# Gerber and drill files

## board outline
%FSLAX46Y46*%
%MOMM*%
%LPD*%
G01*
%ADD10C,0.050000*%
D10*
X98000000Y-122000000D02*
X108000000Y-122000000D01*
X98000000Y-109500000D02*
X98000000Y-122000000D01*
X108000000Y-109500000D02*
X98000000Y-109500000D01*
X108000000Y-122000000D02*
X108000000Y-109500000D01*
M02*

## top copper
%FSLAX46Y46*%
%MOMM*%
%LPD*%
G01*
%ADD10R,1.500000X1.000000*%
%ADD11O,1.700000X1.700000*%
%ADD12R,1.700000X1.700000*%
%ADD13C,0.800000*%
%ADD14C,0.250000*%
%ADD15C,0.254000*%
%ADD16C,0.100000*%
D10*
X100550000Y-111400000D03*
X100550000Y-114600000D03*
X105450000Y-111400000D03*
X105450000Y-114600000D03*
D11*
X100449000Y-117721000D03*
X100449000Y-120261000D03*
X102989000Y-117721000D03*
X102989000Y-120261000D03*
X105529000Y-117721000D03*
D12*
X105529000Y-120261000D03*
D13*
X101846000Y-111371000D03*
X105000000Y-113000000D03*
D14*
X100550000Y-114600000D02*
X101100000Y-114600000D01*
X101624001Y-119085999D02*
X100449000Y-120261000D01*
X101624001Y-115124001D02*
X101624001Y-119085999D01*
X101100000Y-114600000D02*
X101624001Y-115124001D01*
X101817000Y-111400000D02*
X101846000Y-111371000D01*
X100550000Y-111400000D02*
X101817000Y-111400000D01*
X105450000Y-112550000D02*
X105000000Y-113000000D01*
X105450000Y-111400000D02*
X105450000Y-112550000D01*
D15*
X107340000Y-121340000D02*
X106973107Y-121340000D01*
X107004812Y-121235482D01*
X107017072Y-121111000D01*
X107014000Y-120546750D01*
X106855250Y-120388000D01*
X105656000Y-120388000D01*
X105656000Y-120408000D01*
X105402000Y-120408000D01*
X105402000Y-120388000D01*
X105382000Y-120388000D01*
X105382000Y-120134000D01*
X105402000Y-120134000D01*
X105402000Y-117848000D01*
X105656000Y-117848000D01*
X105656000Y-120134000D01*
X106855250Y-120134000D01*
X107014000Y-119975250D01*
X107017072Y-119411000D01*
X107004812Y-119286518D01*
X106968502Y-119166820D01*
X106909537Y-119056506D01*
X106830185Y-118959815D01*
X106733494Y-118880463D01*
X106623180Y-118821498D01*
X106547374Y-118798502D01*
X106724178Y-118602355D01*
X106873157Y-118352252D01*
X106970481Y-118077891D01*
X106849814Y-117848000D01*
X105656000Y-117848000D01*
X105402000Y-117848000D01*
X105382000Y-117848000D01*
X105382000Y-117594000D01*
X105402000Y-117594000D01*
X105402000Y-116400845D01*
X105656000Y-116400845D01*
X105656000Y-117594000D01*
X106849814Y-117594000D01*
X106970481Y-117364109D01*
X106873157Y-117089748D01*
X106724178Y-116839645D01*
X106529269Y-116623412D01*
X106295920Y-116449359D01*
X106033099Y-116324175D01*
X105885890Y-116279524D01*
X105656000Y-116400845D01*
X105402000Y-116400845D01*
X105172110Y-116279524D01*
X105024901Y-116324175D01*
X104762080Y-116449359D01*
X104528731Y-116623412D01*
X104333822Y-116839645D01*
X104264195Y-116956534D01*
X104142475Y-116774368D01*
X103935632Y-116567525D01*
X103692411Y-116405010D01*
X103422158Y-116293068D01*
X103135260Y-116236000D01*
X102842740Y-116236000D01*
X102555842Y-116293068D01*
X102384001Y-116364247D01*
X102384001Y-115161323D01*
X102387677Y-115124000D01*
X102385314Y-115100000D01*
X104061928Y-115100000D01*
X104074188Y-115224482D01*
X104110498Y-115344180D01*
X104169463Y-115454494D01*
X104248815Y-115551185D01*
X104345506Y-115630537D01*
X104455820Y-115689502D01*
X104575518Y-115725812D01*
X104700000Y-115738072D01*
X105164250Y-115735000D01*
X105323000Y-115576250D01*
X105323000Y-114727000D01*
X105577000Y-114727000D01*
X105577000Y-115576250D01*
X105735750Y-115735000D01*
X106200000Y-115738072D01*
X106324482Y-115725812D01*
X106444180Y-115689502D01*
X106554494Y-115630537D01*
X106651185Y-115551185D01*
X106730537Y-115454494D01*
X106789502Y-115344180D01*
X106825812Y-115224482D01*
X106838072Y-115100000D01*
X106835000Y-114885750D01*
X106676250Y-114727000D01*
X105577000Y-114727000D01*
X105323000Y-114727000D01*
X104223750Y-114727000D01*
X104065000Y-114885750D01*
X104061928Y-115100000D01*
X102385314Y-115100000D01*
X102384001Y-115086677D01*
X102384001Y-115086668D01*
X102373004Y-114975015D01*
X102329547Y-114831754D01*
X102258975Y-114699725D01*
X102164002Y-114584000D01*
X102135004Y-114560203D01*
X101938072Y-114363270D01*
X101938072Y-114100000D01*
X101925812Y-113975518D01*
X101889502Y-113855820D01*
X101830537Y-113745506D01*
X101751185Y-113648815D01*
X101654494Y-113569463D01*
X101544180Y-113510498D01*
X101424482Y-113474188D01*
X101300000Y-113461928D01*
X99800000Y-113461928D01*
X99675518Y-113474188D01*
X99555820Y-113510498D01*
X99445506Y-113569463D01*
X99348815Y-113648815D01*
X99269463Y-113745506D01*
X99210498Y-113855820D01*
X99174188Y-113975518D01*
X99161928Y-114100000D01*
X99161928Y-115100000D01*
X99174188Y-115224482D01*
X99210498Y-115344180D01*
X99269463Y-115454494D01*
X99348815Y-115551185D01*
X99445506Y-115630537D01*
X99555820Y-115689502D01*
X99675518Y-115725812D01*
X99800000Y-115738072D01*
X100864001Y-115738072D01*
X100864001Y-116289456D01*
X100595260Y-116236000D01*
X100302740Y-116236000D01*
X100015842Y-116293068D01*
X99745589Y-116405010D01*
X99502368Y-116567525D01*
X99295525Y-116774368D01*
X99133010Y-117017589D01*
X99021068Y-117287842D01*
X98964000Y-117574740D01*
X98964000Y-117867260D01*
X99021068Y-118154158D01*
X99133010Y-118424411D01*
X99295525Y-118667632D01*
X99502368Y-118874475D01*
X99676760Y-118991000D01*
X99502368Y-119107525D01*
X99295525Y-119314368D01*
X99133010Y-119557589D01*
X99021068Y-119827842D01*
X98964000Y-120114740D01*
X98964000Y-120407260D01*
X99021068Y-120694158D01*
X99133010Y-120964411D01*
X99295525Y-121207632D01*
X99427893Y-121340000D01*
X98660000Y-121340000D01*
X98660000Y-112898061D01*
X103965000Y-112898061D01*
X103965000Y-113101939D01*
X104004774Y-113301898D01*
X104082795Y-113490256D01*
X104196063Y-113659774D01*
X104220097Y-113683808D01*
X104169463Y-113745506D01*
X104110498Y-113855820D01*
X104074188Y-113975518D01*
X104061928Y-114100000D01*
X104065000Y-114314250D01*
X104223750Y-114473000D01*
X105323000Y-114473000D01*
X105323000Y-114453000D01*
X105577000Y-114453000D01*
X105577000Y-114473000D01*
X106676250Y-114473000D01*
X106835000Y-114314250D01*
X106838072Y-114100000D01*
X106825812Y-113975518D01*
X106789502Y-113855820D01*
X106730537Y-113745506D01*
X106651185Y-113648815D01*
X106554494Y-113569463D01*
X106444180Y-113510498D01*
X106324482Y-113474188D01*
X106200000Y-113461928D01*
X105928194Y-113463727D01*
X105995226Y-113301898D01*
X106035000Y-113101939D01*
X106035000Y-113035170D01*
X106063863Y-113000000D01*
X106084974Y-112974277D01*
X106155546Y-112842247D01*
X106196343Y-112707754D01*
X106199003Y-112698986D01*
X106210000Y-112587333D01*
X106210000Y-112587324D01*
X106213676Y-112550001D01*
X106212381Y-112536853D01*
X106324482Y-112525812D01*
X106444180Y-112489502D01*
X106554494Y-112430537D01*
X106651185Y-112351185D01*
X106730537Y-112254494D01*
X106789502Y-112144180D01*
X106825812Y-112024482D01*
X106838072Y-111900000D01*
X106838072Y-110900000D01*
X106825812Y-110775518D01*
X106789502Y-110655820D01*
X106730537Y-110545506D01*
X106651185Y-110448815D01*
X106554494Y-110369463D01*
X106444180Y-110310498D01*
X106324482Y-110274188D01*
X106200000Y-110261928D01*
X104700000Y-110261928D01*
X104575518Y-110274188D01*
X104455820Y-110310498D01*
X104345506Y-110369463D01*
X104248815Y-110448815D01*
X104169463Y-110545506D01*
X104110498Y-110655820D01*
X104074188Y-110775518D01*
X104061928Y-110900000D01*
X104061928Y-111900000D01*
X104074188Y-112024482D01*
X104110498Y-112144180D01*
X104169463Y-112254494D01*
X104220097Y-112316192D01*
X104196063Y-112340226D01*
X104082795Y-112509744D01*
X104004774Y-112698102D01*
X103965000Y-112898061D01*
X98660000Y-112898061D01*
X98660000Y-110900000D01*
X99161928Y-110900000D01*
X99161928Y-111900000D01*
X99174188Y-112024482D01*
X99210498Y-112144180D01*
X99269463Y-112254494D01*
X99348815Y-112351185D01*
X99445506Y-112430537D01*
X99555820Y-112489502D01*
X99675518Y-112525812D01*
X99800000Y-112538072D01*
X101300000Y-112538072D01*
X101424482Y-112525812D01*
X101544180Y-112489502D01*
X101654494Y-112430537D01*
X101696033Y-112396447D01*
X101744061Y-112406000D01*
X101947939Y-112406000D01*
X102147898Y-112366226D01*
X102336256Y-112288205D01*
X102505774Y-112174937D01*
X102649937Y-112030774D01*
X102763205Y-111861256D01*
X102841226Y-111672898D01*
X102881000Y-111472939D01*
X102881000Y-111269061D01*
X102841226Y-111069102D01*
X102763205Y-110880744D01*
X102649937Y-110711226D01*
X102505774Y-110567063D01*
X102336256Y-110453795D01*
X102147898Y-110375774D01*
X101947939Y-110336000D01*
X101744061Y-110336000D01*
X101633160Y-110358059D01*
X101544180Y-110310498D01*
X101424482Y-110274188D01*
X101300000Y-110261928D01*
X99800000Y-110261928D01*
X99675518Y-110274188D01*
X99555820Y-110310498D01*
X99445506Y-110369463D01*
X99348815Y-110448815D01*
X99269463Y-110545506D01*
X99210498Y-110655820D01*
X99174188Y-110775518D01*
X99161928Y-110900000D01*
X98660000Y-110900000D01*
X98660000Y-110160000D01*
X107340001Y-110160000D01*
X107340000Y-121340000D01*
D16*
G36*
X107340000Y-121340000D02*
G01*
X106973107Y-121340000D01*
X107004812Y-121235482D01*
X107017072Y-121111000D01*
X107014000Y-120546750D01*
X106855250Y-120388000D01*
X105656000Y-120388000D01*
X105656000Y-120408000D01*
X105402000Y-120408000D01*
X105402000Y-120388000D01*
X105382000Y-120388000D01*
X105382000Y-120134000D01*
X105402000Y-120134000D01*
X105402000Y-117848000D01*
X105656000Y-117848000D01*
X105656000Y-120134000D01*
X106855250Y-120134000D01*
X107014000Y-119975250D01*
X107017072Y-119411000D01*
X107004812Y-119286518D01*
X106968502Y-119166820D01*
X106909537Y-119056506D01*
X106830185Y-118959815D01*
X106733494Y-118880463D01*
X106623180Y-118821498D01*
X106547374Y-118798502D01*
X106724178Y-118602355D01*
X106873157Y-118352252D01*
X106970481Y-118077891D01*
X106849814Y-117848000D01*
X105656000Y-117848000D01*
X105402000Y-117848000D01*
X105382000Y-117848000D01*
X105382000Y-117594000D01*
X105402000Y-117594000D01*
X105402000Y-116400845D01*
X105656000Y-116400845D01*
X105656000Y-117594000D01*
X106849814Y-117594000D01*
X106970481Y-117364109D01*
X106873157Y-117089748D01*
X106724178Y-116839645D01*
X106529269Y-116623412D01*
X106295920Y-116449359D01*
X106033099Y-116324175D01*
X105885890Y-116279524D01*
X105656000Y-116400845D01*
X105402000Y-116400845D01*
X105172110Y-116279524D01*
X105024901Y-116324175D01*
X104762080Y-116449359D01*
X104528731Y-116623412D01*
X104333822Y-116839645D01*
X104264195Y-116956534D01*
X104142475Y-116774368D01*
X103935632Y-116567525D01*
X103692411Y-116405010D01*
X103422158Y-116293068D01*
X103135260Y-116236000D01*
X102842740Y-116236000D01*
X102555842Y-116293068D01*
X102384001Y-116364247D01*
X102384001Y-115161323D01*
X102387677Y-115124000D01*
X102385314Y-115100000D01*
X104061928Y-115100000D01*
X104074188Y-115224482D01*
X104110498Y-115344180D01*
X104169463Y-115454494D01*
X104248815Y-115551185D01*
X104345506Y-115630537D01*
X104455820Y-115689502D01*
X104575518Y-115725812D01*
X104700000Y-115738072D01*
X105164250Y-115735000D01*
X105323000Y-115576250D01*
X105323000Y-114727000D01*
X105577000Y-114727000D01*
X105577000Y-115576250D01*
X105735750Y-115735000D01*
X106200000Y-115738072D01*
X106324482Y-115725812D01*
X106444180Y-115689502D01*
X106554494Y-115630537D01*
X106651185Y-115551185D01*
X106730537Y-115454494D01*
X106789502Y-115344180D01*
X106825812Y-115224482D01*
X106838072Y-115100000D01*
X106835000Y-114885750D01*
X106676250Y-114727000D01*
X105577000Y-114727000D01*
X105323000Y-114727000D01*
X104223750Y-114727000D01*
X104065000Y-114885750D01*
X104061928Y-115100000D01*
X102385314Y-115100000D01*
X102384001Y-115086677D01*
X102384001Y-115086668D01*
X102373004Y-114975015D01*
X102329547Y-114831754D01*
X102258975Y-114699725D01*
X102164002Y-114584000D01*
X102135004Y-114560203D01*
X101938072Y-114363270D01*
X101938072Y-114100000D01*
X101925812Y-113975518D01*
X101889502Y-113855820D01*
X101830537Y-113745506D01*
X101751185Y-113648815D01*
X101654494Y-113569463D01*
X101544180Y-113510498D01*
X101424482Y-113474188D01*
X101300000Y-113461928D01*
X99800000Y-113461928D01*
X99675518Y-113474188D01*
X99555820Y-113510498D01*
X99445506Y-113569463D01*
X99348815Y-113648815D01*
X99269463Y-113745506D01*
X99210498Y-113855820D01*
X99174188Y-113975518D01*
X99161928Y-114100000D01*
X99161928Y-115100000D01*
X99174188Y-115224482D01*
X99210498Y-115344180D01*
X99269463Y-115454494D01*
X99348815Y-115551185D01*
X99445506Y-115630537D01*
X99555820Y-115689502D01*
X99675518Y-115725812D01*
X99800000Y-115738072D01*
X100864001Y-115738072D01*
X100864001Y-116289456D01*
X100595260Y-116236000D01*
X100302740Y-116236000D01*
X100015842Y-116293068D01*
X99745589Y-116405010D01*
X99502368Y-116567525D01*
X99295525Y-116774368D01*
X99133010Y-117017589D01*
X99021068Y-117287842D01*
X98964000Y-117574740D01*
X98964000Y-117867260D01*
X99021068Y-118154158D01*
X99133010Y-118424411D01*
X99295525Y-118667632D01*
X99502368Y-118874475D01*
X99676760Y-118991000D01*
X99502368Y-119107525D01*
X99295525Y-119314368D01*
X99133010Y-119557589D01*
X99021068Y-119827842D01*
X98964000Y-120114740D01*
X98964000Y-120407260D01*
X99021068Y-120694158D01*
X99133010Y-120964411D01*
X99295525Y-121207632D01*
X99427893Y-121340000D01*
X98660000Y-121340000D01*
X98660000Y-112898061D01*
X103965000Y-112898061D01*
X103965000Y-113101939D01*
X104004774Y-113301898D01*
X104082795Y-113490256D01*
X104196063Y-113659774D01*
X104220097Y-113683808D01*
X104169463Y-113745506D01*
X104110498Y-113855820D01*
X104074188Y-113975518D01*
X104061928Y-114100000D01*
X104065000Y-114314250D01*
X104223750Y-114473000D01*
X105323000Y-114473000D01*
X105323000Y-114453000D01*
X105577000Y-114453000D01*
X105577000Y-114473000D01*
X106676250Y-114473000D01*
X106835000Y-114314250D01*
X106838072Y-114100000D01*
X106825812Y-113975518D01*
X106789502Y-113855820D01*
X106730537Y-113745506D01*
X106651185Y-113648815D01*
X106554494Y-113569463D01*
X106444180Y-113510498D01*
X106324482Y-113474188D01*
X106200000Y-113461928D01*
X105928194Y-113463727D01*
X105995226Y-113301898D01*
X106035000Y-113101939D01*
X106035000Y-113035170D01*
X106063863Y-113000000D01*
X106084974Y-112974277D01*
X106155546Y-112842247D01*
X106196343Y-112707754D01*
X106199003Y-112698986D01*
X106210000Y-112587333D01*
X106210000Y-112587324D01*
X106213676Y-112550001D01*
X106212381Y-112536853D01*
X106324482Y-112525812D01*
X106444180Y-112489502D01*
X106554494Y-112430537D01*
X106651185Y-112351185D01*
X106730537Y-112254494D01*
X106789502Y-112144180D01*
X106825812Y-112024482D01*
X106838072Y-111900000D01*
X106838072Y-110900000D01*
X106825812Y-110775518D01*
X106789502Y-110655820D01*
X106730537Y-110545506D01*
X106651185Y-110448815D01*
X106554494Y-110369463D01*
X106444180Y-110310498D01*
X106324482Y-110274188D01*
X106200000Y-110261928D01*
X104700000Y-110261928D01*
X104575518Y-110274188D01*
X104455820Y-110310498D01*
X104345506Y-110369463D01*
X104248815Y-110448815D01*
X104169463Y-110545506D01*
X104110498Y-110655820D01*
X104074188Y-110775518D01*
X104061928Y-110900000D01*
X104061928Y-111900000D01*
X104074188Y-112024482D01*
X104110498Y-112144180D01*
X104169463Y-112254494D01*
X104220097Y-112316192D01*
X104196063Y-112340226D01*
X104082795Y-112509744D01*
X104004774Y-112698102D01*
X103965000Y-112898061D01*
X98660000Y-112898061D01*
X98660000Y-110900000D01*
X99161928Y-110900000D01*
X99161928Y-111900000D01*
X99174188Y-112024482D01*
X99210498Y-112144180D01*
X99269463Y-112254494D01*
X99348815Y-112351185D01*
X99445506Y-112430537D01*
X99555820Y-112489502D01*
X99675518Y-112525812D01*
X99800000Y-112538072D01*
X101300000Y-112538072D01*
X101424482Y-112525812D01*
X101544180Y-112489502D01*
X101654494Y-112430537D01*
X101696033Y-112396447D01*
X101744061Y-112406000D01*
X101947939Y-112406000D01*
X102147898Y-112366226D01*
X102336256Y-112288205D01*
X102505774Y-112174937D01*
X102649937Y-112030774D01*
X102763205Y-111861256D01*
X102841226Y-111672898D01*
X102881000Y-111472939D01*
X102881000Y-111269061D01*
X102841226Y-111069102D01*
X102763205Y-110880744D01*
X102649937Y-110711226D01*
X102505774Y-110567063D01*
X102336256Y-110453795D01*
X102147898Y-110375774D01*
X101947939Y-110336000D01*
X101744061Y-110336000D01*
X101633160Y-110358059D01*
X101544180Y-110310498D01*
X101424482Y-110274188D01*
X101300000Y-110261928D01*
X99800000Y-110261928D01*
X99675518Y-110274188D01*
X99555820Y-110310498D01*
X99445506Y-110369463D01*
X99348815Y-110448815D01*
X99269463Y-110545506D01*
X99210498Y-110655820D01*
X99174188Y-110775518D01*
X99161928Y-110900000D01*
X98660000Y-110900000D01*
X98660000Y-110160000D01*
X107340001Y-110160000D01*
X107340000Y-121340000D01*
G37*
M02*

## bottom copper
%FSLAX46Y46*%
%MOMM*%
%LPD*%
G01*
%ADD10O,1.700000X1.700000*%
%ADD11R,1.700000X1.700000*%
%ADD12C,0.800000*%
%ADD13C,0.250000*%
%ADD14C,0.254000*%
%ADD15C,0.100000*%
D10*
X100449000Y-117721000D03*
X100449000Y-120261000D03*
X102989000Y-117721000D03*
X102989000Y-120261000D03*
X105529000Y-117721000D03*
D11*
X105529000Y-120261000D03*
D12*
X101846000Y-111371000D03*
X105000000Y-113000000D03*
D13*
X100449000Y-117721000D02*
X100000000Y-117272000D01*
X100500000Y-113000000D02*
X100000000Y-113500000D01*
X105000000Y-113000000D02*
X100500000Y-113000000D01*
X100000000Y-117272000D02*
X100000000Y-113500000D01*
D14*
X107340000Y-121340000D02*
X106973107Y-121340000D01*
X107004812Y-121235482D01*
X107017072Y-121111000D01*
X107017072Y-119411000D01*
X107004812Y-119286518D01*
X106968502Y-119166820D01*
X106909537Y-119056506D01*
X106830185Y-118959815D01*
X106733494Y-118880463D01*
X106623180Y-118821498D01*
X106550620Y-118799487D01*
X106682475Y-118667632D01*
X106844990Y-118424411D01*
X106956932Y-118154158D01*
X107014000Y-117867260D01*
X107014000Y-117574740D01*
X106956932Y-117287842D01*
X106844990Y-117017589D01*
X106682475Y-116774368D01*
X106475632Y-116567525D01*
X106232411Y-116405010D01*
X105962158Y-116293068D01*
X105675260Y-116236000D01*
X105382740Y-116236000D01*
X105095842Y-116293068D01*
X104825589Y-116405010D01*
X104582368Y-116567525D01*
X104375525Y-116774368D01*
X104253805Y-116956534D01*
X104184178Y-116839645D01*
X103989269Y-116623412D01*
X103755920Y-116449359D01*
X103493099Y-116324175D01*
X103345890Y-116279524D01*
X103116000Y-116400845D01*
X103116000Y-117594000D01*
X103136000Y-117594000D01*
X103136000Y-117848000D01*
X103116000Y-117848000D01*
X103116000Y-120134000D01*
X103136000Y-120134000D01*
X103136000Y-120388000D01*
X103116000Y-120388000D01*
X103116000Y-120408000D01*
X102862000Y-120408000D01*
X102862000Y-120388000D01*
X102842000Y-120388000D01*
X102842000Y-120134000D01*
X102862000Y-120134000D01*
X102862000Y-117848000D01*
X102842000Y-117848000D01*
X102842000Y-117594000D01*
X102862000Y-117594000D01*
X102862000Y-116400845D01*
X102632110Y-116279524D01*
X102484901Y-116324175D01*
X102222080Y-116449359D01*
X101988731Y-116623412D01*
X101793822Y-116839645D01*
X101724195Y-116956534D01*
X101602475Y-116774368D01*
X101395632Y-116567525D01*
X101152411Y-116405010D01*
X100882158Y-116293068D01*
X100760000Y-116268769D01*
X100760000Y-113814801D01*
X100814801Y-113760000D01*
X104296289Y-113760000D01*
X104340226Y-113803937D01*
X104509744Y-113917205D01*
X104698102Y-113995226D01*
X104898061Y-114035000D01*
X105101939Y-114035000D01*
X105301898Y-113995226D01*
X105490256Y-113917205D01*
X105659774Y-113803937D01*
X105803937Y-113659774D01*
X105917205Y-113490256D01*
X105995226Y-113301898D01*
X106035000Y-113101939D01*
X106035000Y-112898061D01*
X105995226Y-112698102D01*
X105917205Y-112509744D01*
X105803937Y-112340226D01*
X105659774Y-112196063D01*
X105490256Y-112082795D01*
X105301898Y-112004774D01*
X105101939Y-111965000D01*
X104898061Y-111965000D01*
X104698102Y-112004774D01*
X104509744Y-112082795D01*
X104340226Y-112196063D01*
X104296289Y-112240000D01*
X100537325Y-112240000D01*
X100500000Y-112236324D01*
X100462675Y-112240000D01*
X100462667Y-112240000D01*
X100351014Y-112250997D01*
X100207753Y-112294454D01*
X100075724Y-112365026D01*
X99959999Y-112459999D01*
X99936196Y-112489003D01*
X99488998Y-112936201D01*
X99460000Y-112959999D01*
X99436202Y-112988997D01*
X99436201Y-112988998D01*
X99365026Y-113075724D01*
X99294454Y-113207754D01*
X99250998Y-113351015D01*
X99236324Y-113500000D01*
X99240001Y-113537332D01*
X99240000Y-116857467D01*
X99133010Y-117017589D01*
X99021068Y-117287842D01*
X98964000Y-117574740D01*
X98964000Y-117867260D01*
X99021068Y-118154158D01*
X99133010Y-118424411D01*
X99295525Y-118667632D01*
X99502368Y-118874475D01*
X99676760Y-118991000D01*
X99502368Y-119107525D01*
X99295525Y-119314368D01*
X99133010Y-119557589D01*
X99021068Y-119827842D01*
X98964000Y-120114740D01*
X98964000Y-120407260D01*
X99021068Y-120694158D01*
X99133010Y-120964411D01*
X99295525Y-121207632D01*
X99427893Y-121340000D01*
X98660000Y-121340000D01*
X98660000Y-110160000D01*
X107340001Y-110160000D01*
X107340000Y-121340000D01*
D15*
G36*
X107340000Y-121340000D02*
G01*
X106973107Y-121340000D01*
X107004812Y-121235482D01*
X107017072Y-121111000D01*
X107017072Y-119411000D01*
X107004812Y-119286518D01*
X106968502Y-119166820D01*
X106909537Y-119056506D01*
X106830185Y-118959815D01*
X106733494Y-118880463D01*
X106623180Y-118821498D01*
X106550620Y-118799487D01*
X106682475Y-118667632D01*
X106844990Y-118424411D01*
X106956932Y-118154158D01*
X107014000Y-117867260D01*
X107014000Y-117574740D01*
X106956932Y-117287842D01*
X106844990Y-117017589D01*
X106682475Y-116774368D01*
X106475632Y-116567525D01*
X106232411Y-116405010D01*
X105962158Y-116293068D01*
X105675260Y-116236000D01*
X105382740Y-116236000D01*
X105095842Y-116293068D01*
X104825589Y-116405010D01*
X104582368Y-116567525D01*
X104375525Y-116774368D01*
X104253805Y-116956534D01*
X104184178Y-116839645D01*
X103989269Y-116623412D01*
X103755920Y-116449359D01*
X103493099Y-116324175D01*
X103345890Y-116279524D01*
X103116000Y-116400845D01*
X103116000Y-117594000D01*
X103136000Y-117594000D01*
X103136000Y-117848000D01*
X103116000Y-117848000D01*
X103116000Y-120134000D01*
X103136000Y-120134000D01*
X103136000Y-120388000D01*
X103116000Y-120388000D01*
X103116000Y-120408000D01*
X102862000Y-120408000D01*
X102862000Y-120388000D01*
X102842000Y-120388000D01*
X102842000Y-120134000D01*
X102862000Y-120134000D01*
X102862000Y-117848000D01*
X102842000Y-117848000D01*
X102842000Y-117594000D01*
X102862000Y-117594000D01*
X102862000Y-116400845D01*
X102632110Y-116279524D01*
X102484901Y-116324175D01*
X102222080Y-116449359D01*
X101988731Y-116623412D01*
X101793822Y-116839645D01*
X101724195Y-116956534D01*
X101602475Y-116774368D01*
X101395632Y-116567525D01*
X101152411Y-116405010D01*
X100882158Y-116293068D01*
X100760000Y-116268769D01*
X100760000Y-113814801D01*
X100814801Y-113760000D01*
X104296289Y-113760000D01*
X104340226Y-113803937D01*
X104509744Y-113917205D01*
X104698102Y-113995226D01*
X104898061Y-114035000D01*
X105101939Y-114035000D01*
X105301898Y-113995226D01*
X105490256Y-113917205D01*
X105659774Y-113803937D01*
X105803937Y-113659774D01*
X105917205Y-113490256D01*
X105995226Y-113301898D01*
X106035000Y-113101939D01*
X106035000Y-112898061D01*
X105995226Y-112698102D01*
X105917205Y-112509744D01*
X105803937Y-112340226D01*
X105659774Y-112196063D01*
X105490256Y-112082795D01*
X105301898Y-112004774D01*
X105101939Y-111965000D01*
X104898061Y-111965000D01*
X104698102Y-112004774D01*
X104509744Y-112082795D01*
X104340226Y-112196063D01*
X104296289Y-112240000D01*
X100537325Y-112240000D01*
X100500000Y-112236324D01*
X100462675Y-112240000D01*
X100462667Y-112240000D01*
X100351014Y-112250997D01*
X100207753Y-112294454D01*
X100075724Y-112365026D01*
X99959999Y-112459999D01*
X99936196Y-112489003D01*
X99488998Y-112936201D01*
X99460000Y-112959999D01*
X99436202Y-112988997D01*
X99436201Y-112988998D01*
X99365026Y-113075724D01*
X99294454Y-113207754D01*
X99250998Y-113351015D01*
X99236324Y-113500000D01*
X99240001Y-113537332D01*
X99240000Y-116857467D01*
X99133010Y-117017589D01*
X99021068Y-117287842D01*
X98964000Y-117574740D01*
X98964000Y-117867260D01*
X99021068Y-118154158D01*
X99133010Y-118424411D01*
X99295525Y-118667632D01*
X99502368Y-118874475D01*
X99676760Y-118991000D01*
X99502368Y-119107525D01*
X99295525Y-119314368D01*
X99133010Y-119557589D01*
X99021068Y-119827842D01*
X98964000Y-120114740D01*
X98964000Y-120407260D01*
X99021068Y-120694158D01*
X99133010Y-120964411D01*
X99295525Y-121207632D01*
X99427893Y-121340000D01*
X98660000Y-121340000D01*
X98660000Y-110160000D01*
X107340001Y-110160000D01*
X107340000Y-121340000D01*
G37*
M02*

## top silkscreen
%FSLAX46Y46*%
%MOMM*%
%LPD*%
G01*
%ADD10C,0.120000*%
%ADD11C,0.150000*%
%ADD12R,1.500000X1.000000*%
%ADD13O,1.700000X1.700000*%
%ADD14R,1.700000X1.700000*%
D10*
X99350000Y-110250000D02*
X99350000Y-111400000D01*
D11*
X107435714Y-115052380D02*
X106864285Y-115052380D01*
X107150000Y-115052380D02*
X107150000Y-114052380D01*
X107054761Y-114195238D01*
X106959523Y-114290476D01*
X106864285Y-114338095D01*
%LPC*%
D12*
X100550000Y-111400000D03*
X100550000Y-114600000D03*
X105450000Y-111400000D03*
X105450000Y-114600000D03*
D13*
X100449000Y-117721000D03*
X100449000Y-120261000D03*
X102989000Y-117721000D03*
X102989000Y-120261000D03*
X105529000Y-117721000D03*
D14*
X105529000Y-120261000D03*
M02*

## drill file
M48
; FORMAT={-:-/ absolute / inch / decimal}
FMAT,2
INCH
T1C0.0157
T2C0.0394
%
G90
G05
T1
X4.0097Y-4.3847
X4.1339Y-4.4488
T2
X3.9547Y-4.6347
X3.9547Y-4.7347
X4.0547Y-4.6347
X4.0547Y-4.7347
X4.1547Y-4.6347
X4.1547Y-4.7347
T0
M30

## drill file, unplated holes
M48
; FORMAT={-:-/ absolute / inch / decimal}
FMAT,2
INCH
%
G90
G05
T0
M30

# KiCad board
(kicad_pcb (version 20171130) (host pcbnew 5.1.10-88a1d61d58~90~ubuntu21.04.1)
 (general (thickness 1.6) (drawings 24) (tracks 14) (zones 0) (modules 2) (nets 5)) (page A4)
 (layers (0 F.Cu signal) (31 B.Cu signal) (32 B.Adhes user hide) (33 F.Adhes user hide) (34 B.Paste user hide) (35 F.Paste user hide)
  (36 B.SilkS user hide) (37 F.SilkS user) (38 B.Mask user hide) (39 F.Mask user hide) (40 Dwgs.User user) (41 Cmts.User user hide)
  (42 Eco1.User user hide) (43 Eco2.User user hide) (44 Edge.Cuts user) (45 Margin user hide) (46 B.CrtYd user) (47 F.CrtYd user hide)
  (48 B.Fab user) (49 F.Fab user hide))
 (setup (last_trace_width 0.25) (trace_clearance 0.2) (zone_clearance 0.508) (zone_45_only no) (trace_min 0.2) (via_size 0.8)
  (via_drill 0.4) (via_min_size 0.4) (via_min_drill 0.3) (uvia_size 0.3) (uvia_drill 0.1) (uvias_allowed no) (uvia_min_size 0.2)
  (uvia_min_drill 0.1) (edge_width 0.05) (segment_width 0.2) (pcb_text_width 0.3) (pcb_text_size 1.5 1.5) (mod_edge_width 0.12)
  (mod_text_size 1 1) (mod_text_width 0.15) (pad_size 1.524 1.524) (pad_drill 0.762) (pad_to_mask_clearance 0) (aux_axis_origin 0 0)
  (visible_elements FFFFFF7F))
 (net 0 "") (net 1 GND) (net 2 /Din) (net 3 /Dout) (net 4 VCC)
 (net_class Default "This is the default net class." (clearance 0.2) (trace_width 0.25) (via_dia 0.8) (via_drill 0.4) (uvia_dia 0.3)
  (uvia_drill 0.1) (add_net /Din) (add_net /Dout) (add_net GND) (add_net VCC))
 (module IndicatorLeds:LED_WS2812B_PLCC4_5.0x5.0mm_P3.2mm (layer F.Cu) (at 103 113 180)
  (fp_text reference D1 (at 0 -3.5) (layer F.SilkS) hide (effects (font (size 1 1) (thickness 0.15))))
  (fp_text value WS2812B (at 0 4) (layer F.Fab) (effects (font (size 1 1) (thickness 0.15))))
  (fp_line (start 3.65 2.75) (end 3.65 1.6) (layer F.SilkS) (width 0.12))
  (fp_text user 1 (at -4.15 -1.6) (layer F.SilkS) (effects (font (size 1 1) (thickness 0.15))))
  (pad 3 smd rect (at 2.45 1.6 180) (size 1.5 1) (layers F.Cu F.Paste F.Mask) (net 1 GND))
  (pad 4 smd rect (at 2.45 -1.6 180) (size 1.5 1) (layers F.Cu F.Paste F.Mask) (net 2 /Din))
  (pad 2 smd rect (at -2.45 1.6 180) (size 1.5 1) (layers F.Cu F.Paste F.Mask) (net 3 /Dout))
  (pad 1 smd rect (at -2.45 -1.6 180) (size 1.5 1) (layers F.Cu F.Paste F.Mask) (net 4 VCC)))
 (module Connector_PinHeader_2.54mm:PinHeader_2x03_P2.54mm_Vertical (layer B.Cu) (at 105.529 120.261 90)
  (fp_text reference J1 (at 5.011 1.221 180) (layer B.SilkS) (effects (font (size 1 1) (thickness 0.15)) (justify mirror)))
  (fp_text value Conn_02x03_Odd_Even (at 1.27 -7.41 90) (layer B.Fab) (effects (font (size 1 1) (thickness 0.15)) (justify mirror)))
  (pad 6 thru_hole oval (at 2.54 -5.08 90) (size 1.7 1.7) (drill 1) (layers *.Cu *.Mask) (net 3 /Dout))
  (pad 5 thru_hole oval (at 0 -5.08 90) (size 1.7 1.7) (drill 1) (layers *.Cu *.Mask) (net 2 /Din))
  (pad 4 thru_hole oval (at 2.54 -2.54 90) (size 1.7 1.7) (drill 1) (layers *.Cu *.Mask) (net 1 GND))
  (pad 3 thru_hole oval (at 0 -2.54 90) (size 1.7 1.7) (drill 1) (layers *.Cu *.Mask) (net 1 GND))
  (pad 2 thru_hole oval (at 2.54 0 90) (size 1.7 1.7) (drill 1) (layers *.Cu *.Mask) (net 4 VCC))
  (pad 1 thru_hole rect (at 0 0 90) (size 1.7 1.7) (drill 1) (layers *.Cu *.Mask) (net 4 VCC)))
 (gr_line (start 98 122) (end 108 122) (layer Edge.Cuts) (width 0.05))
 (gr_line (start 98 109.5) (end 98 122) (layer Edge.Cuts) (width 0.05))
 (gr_line (start 108 109.5) (end 98 109.5) (layer Edge.Cuts) (width 0.05))
 (gr_line (start 108 122) (end 108 109.5) (layer Edge.Cuts) (width 0.05))
 (segment (start 100.55 114.6) (end 101.1 114.6) (width 0.25) (layer F.Cu) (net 2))
 (segment (start 101.624001 119.085999) (end 100.449 120.261) (width 0.25) (layer F.Cu) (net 2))
 (segment (start 101.624001 115.124001) (end 101.624001 119.085999) (width 0.25) (layer F.Cu) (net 2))
 (segment (start 101.1 114.6) (end 101.624001 115.124001) (width 0.25) (layer F.Cu) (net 2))
 (via (at 101.846 111.371) (size 0.8) (drill 0.4) (layers F.Cu B.Cu) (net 1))
 (segment (start 101.817 111.4) (end 101.846 111.371) (width 0.25) (layer F.Cu) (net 1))
 (segment (start 100.55 111.4) (end 101.817 111.4) (width 0.25) (layer F.Cu) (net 1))
 (segment (start 100.449 117.721) (end 100 117.272) (width 0.25) (layer B.Cu) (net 3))
 (via (at 105 113) (size 0.8) (drill 0.4) (layers F.Cu B.Cu) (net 3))
 (segment (start 105.45 112.55) (end 105 113) (width 0.25) (layer F.Cu) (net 3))
 (segment (start 105.45 111.4) (end 105.45 112.55) (width 0.25) (layer F.Cu) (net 3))
 (segment (start 100.5 113) (end 100 113.5) (width 0.25) (layer B.Cu) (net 3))
 (segment (start 105 113) (end 100.5 113) (width 0.25) (layer B.Cu) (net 3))
 (segment (start 100 117.272) (end 100 113.5) (width 0.25) (layer B.Cu) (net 3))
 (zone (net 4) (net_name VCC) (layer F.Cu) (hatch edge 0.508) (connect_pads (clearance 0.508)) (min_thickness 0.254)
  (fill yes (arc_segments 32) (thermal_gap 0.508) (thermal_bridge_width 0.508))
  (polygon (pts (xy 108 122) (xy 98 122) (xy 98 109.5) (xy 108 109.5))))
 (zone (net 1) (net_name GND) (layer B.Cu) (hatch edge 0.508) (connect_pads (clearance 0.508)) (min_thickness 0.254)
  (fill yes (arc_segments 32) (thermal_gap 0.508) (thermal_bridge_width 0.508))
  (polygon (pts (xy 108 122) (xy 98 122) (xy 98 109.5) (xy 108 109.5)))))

